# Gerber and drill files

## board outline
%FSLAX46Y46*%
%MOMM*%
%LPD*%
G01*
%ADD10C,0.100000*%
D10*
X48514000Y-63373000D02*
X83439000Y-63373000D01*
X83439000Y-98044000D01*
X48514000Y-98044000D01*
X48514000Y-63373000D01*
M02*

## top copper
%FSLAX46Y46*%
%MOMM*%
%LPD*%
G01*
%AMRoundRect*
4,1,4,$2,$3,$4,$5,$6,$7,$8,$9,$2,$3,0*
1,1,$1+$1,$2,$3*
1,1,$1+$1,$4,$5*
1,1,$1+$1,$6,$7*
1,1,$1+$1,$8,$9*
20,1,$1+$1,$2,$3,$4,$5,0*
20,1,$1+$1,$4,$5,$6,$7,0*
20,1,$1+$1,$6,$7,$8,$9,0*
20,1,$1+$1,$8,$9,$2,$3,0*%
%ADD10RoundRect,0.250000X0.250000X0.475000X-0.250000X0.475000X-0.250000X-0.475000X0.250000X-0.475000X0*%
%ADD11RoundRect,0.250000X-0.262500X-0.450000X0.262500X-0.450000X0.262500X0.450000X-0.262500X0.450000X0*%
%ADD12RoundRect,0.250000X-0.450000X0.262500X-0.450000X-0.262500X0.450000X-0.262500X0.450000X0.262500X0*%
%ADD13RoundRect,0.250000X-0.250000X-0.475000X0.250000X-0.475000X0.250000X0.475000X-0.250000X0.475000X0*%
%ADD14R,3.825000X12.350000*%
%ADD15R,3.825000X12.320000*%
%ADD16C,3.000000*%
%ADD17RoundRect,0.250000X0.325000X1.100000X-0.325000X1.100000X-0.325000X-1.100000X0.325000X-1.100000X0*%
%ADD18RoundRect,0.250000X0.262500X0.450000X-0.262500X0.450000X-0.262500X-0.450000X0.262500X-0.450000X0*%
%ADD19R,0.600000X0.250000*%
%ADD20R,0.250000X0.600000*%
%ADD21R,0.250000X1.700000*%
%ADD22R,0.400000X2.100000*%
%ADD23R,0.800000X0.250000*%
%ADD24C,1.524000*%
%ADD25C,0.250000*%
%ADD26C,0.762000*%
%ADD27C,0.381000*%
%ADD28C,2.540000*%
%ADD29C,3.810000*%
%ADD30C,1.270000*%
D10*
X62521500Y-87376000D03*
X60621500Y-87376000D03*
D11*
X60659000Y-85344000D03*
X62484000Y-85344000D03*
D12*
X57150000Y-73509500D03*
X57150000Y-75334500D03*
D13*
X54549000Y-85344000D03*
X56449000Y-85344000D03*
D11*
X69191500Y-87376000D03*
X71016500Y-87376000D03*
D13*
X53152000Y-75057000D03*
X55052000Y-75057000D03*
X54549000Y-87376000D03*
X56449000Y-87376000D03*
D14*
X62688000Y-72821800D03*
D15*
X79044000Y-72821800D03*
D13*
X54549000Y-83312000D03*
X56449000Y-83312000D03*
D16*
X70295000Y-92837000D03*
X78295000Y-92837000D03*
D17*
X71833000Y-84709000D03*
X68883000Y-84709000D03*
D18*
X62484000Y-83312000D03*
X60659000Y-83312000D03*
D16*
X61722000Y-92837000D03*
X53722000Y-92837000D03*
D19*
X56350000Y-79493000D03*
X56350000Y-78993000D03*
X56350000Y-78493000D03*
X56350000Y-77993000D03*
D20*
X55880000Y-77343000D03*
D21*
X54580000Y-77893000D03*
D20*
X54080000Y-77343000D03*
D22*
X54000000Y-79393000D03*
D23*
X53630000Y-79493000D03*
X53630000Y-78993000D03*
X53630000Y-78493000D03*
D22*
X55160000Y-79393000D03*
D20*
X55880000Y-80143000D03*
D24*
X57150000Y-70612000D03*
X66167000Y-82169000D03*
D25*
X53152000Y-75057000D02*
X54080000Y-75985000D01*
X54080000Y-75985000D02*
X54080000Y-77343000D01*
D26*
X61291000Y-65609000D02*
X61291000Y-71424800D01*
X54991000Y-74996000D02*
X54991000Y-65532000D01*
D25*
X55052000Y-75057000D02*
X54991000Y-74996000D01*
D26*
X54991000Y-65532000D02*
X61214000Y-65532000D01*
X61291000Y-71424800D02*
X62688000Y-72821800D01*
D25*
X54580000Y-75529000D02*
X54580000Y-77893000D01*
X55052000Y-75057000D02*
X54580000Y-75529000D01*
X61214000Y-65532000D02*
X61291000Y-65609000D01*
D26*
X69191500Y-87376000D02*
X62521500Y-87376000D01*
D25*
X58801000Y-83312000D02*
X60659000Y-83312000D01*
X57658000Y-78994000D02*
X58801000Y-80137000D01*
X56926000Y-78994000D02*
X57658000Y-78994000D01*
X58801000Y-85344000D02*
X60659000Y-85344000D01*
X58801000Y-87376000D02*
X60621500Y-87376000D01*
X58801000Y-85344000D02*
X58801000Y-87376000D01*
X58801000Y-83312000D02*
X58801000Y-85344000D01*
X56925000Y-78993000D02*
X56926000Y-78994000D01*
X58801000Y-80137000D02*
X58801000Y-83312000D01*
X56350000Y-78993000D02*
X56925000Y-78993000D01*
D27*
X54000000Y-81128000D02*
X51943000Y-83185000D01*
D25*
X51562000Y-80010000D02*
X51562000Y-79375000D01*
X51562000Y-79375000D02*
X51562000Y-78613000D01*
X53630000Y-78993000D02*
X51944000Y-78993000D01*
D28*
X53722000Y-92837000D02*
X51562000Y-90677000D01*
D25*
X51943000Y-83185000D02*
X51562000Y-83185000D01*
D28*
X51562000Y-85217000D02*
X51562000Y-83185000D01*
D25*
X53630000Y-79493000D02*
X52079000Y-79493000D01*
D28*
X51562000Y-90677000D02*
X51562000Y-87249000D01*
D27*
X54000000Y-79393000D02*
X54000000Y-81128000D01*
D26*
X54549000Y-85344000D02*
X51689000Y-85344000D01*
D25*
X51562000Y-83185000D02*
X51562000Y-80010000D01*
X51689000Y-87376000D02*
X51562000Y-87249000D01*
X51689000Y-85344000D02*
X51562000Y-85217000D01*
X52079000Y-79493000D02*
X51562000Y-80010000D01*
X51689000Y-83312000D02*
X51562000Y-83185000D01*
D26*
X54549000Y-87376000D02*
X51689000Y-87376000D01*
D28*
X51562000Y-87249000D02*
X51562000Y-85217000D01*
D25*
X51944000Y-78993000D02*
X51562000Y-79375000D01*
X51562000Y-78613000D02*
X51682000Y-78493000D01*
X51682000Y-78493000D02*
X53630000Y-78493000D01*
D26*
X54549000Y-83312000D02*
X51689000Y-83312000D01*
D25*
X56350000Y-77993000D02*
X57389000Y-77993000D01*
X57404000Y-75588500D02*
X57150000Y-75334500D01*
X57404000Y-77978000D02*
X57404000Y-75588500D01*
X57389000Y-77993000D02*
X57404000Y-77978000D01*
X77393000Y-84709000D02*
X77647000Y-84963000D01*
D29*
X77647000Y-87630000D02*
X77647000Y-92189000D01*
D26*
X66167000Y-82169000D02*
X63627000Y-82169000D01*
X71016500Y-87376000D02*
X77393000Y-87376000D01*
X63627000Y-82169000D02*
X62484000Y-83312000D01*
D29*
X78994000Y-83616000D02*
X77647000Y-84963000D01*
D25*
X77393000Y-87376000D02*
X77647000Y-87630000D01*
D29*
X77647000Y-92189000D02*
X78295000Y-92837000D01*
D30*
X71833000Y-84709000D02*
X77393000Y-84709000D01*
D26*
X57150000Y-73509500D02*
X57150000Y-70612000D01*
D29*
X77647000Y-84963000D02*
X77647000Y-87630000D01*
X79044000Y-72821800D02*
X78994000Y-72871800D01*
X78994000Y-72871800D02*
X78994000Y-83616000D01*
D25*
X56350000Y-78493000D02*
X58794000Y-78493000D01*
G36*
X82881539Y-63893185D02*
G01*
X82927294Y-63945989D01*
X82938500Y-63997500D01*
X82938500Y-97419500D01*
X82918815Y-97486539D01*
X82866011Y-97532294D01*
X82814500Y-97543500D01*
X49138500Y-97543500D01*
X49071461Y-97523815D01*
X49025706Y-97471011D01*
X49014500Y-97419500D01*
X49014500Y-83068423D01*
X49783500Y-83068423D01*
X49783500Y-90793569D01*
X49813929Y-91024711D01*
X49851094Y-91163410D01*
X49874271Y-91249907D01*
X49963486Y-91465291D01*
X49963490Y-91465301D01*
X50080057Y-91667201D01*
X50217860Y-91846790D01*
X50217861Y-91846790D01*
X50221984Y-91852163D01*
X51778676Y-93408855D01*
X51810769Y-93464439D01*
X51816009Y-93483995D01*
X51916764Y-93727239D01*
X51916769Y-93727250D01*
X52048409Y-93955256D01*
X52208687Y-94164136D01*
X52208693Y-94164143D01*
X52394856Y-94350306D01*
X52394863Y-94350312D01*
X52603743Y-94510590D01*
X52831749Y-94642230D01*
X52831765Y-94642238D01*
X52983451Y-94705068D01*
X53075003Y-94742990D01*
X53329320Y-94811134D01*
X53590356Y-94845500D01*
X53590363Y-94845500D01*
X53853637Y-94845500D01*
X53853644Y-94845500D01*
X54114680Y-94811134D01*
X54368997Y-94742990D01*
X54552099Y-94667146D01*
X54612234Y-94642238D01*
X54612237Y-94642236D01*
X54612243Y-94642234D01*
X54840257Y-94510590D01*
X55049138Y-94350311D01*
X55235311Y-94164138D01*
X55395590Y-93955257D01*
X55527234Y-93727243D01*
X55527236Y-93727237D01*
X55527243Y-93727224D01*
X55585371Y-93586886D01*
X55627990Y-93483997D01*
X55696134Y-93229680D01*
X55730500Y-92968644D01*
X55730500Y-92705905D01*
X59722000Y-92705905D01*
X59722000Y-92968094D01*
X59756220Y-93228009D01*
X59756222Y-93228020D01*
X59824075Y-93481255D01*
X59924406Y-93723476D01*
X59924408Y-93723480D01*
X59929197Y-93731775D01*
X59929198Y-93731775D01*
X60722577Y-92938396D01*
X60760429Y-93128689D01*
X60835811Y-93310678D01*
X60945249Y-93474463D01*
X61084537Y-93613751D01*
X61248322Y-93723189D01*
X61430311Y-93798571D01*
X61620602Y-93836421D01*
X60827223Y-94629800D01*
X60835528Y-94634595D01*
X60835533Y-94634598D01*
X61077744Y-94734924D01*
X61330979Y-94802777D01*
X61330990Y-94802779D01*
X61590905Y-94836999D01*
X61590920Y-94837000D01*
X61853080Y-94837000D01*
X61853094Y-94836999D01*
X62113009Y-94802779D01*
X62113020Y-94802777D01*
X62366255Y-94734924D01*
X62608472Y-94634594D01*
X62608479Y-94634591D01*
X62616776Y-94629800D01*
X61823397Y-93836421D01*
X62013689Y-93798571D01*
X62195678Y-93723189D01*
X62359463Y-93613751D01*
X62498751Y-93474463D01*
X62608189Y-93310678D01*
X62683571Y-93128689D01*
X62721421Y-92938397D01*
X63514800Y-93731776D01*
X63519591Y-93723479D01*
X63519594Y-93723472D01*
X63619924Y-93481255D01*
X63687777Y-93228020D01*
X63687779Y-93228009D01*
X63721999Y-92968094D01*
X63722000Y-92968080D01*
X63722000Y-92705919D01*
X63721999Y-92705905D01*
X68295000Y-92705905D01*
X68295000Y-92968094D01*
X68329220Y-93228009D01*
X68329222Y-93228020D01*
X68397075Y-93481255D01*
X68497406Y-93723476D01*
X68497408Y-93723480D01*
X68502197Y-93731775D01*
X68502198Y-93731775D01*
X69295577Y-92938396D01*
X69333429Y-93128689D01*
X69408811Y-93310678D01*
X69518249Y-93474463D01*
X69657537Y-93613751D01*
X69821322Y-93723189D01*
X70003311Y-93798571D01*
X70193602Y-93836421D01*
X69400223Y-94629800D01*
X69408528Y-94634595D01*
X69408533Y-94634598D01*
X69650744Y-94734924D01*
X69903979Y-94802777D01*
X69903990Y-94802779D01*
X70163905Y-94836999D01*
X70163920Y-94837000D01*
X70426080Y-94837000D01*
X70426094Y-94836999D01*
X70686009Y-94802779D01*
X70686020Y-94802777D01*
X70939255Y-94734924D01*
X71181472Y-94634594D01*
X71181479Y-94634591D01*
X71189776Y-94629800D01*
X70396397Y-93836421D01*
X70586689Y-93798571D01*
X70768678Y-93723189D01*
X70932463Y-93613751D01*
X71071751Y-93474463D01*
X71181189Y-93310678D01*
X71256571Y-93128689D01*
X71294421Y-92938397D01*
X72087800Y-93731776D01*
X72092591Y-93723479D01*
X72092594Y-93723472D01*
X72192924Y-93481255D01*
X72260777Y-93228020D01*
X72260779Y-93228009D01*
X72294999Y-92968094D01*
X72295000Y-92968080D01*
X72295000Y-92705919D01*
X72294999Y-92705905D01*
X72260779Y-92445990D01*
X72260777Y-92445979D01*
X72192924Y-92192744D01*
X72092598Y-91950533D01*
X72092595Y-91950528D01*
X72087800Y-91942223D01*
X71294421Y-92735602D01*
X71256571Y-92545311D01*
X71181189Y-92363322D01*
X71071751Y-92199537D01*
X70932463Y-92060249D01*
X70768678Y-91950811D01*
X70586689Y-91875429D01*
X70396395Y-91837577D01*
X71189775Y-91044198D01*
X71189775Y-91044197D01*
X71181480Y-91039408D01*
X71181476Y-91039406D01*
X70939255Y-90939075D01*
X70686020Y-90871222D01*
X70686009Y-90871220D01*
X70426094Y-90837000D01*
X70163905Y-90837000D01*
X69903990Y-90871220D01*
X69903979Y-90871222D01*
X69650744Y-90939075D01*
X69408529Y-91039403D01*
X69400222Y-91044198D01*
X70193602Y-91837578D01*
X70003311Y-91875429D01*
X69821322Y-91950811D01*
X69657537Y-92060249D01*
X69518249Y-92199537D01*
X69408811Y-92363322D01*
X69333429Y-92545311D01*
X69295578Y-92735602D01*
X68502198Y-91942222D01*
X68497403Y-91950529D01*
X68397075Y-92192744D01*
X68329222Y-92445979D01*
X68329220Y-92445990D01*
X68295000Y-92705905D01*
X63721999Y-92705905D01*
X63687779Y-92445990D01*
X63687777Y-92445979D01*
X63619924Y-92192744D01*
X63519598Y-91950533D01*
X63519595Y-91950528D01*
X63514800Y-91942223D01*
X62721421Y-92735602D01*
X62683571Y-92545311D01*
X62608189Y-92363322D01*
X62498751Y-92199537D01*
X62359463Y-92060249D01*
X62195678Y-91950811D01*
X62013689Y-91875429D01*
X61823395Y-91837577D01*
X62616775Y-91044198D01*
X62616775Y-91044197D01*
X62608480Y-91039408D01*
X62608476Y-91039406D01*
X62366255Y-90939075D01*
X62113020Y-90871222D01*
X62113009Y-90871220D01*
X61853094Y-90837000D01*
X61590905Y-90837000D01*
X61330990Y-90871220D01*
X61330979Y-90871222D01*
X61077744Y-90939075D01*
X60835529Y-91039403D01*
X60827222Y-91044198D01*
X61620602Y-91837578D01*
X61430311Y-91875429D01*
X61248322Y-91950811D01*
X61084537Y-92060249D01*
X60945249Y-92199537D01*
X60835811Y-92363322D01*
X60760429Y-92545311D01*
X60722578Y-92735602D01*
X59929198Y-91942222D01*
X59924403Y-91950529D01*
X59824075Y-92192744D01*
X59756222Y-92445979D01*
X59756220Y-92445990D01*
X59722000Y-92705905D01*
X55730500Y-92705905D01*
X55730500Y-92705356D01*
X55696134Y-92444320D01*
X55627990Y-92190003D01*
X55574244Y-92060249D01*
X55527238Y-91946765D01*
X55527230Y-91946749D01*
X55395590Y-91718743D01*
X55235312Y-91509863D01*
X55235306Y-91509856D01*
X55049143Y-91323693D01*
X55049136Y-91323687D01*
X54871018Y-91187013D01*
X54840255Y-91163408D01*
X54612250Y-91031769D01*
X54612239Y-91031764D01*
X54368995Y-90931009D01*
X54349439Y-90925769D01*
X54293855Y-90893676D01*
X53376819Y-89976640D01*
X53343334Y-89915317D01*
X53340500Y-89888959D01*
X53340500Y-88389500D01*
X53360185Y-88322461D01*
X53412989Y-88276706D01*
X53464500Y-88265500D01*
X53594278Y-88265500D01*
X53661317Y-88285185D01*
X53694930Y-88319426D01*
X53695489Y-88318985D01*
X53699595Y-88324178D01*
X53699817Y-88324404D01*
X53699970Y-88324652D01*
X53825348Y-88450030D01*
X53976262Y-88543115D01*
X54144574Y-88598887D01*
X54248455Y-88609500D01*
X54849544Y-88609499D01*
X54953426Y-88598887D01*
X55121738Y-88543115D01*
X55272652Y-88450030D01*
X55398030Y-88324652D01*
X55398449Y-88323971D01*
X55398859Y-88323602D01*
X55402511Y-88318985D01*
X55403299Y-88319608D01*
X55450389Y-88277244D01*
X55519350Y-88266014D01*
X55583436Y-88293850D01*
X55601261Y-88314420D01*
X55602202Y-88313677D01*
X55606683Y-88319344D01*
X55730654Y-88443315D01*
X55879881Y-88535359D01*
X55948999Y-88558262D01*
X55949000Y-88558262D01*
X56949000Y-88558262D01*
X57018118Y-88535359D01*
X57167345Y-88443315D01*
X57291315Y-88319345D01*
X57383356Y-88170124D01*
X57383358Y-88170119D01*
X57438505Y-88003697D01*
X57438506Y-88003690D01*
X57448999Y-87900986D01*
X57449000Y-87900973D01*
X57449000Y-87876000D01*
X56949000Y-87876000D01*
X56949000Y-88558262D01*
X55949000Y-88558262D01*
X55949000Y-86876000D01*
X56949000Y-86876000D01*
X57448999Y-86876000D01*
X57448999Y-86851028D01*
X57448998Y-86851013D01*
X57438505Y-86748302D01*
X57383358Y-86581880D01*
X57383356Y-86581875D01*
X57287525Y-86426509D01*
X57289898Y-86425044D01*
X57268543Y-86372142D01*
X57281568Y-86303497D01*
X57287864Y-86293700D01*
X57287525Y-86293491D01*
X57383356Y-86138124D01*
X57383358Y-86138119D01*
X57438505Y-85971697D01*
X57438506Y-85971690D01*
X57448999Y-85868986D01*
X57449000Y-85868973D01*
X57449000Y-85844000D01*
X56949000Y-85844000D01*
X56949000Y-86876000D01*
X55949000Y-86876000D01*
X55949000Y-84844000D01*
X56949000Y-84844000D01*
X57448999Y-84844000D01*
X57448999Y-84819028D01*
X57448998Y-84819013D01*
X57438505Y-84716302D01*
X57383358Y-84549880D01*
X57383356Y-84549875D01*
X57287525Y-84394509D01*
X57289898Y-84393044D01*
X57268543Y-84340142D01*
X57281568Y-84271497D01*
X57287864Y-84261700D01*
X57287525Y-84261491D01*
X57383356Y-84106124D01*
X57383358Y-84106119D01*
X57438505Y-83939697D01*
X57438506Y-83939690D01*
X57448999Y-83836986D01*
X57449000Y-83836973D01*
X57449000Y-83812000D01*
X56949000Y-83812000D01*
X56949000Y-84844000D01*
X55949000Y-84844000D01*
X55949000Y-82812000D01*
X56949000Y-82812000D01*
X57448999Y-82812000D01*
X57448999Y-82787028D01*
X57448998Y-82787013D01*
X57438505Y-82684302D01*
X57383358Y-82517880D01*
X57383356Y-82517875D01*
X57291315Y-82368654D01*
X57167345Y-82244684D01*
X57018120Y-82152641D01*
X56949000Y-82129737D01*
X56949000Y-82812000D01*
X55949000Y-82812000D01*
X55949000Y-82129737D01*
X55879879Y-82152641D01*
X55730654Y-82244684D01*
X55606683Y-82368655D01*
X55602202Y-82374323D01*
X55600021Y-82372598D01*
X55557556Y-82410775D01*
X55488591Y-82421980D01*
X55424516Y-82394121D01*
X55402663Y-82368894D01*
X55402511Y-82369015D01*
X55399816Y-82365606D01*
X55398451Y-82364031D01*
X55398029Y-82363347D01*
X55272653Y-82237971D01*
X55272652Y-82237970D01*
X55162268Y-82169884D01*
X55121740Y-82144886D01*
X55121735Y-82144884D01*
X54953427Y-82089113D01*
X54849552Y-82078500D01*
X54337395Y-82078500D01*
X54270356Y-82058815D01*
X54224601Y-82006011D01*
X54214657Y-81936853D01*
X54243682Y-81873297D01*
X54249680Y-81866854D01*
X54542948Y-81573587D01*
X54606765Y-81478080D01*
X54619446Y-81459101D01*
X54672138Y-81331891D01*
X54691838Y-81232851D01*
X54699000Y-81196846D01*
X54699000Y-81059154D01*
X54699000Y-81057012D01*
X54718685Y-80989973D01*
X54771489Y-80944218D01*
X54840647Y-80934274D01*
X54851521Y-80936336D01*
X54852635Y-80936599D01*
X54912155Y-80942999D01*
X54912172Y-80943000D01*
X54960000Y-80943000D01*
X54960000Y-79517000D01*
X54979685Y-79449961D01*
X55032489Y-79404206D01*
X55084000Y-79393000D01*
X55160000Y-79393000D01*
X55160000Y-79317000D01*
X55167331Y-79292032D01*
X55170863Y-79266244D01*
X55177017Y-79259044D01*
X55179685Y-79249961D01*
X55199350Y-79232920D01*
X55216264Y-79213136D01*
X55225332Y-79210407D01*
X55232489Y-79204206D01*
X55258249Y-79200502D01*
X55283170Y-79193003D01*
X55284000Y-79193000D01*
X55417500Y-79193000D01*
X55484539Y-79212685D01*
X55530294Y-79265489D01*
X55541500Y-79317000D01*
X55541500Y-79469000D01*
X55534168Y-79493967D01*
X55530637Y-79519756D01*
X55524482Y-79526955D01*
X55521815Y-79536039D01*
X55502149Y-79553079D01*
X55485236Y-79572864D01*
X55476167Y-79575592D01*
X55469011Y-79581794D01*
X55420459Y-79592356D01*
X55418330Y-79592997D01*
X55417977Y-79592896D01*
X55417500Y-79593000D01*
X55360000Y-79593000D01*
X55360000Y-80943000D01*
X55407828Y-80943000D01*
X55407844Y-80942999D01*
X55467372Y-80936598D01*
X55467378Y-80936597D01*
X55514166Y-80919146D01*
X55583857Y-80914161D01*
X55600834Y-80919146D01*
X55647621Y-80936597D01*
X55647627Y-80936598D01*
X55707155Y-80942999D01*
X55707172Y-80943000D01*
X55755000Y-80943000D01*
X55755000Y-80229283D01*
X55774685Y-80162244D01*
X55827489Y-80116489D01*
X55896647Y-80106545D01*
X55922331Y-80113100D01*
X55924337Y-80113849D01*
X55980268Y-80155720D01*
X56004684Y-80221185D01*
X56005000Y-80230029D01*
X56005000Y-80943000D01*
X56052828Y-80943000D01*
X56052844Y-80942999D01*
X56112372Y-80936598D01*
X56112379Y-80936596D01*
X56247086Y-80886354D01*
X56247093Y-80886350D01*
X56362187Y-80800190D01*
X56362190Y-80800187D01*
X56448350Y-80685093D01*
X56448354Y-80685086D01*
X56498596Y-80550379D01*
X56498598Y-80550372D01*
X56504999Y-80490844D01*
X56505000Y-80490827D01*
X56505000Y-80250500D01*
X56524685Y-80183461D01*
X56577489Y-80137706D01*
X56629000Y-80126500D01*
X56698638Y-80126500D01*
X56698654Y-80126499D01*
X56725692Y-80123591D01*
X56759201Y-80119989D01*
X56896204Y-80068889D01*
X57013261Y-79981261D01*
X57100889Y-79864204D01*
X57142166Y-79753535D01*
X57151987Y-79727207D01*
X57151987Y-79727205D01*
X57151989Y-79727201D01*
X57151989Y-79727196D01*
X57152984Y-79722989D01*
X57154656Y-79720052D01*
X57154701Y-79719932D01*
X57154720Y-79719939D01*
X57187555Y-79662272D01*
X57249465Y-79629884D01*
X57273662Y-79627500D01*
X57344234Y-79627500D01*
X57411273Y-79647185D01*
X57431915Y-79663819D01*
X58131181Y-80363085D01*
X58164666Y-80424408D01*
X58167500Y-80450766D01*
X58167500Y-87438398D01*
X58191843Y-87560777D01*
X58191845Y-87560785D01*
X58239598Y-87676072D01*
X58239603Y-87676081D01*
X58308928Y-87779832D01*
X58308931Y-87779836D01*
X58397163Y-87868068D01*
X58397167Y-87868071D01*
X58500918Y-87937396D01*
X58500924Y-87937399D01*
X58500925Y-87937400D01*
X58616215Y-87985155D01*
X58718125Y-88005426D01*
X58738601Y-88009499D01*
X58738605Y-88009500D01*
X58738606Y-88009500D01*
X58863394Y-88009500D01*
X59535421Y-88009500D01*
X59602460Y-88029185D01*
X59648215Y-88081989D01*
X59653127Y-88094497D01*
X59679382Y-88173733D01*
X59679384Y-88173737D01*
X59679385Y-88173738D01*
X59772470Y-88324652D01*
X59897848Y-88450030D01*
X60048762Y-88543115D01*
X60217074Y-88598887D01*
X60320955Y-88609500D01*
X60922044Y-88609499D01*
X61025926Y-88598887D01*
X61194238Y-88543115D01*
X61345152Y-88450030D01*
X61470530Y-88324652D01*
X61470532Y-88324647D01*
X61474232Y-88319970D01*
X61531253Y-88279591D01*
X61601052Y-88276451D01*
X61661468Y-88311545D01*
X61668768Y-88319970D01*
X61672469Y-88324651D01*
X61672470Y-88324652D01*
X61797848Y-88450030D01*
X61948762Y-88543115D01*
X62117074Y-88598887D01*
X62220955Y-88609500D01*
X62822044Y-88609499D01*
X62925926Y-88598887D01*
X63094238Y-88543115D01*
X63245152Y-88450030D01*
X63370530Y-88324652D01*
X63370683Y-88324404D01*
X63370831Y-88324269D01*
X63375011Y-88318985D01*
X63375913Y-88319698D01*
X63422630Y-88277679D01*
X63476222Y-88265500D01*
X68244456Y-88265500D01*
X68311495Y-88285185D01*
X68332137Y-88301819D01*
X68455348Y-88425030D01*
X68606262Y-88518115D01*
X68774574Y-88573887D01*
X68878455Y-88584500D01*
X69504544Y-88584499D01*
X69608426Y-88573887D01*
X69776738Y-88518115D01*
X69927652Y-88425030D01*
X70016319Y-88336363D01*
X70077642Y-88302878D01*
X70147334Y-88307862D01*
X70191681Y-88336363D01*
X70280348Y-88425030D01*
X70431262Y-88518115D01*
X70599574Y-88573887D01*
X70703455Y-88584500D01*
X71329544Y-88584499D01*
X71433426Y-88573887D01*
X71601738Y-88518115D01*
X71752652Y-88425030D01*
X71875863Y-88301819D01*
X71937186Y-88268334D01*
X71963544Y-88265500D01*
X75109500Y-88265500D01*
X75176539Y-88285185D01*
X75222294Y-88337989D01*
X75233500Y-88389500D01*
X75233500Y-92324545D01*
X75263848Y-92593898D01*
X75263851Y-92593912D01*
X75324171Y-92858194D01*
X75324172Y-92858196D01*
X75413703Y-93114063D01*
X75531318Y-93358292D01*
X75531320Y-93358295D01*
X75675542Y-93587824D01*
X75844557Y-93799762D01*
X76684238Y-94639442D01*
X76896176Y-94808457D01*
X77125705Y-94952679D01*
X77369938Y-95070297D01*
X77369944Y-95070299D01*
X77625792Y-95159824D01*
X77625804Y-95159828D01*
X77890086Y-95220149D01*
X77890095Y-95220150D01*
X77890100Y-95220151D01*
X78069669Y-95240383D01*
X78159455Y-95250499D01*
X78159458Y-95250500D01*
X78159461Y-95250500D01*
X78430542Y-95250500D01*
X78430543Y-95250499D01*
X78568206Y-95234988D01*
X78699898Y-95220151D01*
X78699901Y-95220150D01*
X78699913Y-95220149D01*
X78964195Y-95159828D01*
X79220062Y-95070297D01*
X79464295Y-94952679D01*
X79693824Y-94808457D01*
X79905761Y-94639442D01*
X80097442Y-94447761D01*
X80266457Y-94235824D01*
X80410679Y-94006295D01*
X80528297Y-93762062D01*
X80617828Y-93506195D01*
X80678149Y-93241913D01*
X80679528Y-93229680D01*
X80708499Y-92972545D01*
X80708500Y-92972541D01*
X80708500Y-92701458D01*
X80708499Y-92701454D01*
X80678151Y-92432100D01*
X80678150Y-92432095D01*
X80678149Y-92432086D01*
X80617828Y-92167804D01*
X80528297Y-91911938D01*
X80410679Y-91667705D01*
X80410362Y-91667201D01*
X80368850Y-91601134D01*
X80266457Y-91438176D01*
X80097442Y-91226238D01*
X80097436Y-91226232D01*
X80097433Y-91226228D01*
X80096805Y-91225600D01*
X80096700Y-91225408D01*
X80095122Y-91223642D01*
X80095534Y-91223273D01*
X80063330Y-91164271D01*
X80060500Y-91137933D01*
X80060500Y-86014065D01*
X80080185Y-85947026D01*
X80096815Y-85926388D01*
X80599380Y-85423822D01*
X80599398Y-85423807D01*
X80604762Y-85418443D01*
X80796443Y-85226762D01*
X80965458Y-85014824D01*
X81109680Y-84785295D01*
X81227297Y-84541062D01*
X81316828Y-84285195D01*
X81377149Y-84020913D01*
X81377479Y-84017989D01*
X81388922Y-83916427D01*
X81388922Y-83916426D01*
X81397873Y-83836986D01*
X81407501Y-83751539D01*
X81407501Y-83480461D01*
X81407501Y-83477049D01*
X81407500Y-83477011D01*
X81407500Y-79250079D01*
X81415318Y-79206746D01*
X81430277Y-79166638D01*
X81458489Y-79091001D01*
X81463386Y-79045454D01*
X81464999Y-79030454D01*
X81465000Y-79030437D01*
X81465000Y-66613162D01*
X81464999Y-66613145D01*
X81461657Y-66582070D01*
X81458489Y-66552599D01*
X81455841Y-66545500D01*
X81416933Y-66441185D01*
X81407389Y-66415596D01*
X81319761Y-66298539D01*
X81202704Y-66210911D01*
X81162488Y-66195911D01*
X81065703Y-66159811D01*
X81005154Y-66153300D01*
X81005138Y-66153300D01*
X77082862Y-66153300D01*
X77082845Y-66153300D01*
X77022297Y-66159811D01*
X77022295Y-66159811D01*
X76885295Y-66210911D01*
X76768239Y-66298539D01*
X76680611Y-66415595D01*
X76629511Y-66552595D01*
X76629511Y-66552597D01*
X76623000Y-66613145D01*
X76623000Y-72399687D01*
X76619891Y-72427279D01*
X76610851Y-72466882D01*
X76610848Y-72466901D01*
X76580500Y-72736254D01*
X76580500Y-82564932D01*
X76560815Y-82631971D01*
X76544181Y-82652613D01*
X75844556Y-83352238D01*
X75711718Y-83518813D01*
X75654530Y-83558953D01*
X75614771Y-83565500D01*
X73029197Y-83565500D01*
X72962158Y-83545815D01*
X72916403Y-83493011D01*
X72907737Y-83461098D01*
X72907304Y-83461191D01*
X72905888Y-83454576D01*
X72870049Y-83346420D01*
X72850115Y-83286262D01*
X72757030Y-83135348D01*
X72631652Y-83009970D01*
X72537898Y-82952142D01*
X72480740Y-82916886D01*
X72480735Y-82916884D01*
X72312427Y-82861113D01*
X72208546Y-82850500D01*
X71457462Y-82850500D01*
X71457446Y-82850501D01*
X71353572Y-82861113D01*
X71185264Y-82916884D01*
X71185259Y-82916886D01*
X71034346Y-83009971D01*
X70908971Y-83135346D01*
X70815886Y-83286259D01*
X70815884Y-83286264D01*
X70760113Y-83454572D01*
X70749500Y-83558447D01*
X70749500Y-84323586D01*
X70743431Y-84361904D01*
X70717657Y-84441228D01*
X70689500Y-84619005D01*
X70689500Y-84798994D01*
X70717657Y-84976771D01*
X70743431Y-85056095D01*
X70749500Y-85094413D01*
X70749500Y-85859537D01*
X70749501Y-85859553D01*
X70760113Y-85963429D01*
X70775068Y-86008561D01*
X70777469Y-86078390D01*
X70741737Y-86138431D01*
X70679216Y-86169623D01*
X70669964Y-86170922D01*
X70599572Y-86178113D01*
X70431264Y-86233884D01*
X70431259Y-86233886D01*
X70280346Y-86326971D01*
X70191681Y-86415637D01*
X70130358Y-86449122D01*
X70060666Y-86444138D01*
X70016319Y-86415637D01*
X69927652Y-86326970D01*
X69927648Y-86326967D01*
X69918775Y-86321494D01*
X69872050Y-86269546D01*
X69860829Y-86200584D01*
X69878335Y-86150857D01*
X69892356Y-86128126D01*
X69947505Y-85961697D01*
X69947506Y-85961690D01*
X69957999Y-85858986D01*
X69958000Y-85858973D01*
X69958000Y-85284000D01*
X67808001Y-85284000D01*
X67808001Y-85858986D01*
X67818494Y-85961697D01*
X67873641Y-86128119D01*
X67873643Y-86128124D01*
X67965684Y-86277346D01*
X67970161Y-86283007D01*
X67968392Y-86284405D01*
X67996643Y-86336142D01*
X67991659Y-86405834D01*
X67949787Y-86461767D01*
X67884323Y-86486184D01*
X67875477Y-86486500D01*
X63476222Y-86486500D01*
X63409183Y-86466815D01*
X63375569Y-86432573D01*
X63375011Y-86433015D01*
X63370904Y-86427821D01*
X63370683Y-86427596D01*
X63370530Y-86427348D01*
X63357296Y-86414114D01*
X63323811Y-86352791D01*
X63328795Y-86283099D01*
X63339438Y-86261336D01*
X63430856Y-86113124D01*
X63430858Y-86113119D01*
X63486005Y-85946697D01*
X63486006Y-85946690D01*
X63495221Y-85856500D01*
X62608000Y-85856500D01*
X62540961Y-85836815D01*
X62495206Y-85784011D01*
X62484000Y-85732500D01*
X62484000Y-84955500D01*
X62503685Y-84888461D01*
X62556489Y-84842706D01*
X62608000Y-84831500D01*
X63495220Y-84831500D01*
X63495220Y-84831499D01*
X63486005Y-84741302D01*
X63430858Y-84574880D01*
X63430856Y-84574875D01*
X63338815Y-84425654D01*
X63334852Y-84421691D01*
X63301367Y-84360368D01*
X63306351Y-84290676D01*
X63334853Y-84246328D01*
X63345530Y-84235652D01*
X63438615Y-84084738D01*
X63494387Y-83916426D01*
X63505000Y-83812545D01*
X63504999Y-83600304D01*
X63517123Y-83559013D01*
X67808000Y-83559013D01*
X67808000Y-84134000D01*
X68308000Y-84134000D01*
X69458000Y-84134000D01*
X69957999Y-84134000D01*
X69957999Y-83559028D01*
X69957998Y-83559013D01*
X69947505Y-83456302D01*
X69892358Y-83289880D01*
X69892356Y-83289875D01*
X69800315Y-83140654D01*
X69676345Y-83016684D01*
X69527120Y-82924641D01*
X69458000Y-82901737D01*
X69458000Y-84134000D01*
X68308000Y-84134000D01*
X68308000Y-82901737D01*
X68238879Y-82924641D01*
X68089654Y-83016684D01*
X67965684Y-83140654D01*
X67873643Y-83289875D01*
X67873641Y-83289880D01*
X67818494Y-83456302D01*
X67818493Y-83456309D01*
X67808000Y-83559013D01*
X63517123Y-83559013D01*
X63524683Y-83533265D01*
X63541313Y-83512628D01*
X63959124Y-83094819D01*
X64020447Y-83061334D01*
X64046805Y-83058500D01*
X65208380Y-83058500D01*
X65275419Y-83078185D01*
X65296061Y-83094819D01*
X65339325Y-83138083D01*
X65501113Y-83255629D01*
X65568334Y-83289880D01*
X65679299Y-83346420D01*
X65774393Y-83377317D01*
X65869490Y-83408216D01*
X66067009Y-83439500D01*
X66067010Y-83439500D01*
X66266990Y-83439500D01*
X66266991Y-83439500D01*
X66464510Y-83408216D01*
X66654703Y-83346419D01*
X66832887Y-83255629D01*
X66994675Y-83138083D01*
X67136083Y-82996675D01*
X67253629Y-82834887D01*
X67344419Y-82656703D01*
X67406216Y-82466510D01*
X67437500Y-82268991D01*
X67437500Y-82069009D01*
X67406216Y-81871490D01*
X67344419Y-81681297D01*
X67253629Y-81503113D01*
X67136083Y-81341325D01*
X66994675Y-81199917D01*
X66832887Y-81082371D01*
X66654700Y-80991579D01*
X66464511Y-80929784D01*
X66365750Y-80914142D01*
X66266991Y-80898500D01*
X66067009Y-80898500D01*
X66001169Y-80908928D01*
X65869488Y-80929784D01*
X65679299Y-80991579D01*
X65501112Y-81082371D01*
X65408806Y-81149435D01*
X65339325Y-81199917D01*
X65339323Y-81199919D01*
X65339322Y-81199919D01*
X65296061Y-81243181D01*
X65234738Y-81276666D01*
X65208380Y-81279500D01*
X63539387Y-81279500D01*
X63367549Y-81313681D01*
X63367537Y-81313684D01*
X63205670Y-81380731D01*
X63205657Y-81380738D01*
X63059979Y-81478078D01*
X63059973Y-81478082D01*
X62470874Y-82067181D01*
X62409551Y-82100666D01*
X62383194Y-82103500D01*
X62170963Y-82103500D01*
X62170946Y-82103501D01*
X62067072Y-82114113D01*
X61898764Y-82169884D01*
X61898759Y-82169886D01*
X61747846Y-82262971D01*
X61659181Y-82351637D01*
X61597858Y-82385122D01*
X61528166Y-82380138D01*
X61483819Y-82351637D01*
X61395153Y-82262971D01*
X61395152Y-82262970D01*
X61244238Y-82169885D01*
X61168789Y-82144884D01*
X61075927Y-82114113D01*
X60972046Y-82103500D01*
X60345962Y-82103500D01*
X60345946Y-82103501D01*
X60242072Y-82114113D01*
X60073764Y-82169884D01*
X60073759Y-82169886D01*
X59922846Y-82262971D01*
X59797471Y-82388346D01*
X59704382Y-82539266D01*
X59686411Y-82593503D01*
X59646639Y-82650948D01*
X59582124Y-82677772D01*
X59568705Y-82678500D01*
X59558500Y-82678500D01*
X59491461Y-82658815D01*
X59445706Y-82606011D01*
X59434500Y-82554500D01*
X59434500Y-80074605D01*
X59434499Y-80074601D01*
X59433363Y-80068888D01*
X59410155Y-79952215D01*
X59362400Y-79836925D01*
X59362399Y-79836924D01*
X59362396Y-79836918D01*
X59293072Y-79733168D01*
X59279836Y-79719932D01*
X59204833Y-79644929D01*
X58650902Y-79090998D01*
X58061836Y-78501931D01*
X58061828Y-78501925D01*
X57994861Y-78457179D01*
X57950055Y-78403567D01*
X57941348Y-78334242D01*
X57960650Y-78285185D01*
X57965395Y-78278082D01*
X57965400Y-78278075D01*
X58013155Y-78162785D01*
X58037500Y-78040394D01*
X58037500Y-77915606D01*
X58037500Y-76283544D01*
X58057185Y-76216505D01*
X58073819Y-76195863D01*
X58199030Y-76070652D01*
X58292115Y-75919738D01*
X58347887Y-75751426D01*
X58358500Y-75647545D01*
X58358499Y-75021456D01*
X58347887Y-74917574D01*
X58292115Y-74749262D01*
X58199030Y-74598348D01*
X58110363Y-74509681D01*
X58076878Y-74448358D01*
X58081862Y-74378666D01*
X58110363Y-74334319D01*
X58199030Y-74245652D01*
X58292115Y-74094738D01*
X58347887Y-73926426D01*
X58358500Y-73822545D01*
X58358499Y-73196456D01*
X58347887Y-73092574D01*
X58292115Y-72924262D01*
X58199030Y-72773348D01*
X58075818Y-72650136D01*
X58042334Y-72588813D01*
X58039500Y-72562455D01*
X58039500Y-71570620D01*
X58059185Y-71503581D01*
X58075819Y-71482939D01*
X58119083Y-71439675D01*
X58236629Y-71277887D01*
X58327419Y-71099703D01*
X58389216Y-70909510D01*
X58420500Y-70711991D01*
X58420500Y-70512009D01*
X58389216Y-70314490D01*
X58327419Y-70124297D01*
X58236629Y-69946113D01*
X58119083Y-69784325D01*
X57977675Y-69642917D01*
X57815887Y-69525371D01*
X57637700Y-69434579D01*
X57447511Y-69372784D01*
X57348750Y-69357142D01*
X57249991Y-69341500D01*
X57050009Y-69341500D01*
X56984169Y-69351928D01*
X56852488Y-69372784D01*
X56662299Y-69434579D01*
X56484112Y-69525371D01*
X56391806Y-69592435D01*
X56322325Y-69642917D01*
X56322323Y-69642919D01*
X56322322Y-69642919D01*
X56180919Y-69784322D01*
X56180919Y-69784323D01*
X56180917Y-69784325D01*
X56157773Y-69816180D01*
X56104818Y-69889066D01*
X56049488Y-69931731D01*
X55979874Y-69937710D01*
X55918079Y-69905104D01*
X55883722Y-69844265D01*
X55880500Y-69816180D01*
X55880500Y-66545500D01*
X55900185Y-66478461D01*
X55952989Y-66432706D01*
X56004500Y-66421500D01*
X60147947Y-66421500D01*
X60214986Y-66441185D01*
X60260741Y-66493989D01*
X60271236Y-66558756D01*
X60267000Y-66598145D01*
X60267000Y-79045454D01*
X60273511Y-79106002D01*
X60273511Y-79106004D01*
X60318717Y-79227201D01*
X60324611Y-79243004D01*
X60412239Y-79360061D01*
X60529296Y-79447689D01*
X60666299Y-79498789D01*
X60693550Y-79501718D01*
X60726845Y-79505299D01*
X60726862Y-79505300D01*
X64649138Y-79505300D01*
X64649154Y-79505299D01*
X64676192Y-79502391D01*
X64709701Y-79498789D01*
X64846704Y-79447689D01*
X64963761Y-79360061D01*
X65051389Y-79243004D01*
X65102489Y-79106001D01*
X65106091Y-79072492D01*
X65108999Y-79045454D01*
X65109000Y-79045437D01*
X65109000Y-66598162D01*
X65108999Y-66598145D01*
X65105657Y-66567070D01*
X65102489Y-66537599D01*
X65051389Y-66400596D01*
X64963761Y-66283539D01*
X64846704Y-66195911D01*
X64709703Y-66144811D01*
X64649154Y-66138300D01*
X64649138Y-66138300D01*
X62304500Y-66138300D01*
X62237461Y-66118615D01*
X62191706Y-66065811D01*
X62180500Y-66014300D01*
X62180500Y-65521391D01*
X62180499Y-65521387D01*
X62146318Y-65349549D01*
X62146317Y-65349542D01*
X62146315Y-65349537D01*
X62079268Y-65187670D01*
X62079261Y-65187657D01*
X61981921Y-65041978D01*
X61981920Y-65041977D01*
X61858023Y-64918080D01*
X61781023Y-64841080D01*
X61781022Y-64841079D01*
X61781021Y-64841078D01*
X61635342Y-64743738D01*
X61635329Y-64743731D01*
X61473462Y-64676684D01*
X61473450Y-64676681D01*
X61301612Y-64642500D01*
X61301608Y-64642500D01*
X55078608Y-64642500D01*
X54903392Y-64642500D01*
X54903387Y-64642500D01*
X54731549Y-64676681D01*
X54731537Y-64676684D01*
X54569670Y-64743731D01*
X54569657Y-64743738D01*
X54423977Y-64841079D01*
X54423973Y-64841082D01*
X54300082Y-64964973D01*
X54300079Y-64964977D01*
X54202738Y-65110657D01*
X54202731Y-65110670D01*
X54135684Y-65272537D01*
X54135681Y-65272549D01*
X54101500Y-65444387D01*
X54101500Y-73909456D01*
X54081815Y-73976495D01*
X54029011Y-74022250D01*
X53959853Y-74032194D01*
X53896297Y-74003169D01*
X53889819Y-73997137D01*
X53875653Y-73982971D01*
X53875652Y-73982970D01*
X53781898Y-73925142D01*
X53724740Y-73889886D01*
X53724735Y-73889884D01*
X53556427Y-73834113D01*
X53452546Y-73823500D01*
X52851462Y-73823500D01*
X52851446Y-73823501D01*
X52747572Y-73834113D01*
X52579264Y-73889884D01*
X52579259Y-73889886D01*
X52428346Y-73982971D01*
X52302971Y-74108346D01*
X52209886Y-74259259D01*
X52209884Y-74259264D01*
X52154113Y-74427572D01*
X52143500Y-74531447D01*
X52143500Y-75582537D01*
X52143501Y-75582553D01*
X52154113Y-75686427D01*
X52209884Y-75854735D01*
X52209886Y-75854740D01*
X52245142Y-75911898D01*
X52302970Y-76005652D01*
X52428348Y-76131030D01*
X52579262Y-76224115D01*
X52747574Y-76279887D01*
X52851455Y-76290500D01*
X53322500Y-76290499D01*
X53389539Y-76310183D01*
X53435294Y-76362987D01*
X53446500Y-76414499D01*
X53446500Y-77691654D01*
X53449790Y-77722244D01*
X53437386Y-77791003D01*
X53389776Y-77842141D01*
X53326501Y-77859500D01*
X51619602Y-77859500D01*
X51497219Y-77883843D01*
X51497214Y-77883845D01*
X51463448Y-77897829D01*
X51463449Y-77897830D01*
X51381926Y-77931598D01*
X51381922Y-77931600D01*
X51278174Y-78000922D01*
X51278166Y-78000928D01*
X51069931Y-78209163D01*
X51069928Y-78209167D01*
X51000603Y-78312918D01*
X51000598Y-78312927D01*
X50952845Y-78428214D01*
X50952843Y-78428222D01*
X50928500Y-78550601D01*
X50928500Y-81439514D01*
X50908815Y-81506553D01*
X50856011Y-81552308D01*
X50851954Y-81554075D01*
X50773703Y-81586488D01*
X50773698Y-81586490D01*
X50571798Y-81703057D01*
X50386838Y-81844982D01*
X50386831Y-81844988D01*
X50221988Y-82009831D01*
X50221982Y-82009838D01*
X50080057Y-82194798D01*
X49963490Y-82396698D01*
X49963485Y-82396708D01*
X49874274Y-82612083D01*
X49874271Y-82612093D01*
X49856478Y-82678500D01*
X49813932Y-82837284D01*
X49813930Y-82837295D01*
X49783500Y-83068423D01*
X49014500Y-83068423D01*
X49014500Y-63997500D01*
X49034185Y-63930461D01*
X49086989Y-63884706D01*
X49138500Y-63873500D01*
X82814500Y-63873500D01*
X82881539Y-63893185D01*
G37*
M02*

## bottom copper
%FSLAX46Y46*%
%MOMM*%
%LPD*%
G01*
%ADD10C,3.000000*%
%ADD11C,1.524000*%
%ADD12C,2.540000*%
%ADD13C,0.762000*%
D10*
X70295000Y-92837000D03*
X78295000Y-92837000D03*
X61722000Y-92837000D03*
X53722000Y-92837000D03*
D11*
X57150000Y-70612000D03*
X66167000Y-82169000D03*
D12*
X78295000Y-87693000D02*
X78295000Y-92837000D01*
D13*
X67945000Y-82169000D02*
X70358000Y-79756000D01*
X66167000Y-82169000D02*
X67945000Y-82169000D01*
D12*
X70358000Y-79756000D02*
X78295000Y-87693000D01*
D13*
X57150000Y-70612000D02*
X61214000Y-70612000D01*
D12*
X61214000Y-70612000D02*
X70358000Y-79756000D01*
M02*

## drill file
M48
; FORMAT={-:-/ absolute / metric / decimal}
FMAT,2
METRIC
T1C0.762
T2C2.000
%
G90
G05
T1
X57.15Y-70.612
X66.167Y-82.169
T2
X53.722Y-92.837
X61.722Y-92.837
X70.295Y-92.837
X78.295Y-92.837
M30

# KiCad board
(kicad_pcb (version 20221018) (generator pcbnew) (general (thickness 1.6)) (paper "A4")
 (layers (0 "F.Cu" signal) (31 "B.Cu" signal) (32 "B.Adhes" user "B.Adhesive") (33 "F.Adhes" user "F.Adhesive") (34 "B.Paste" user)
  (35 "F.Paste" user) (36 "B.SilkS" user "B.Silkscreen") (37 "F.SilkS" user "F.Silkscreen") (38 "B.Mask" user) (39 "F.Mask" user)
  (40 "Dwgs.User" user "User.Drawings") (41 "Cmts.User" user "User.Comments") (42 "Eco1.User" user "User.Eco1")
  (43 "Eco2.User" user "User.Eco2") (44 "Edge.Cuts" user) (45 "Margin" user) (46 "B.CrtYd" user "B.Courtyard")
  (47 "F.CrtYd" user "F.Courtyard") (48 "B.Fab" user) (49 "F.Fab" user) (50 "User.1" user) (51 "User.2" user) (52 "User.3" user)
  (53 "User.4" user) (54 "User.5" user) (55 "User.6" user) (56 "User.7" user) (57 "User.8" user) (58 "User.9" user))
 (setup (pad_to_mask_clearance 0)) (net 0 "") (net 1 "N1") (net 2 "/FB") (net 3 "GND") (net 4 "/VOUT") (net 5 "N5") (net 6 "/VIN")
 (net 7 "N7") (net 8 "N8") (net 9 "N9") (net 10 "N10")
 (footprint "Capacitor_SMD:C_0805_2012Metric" (layer "F.Cu") (at 61.5715 87.376 180)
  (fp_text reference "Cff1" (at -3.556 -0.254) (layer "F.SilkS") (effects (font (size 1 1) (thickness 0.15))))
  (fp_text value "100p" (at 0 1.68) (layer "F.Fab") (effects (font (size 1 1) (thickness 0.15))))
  (pad "1" smd roundrect (at -0.95 0 180) (size 1 1.45) (layers "F.Cu" "F.Paste" "F.Mask") (roundrect_rratio 0.25) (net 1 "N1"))
  (pad "2" smd roundrect (at 0.95 0 180) (size 1 1.45) (layers "F.Cu" "F.Paste" "F.Mask") (roundrect_rratio 0.25) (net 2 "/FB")))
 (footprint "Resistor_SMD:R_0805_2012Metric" (layer "F.Cu") (at 61.5715 85.344)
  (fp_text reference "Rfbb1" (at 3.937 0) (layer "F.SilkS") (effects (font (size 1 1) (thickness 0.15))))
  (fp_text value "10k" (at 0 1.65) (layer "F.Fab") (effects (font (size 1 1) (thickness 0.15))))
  (pad "1" smd roundrect (at -0.9125 0) (size 1.025 1.4) (layers "F.Cu" "F.Paste" "F.Mask") (roundrect_rratio 0.243902) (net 2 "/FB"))
  (pad "2" smd roundrect (at 0.9125 0) (size 1.025 1.4) (layers "F.Cu" "F.Paste" "F.Mask") (roundrect_rratio 0.243902) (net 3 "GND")))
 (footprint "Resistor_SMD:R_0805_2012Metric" (layer "F.Cu") (at 57.15 74.422 -90)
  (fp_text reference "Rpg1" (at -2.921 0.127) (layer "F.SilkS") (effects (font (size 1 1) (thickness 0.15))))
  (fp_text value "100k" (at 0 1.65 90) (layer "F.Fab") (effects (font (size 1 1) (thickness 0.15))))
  (pad "1" smd roundrect (at -0.9125 0 270) (size 1.025 1.4) (layers "F.Cu" "F.Paste" "F.Mask") (roundrect_rratio 0.243902) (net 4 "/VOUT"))
  (pad "2" smd roundrect (at 0.9125 0 270) (size 1.025 1.4) (layers "F.Cu" "F.Paste" "F.Mask") (roundrect_rratio 0.243902) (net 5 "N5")))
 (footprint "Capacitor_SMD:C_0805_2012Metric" (layer "F.Cu") (at 55.499 85.344)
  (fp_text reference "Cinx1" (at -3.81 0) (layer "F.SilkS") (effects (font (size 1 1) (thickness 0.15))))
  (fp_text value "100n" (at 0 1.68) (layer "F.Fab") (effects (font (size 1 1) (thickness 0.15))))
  (pad "1" smd roundrect (at -0.95 0) (size 1 1.45) (layers "F.Cu" "F.Paste" "F.Mask") (roundrect_rratio 0.25) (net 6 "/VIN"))
  (pad "2" smd roundrect (at 0.95 0) (size 1 1.45) (layers "F.Cu" "F.Paste" "F.Mask") (roundrect_rratio 0.25) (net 3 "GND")))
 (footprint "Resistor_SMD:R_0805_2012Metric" (layer "F.Cu") (at 70.104 87.376)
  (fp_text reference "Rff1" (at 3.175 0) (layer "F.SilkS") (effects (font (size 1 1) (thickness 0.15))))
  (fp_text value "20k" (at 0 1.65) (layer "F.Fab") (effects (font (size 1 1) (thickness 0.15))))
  (pad "1" smd roundrect (at -0.9125 0) (size 1.025 1.4) (layers "F.Cu" "F.Paste" "F.Mask") (roundrect_rratio 0.243902) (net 1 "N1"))
  (pad "2" smd roundrect (at 0.9125 0) (size 1.025 1.4) (layers "F.Cu" "F.Paste" "F.Mask") (roundrect_rratio 0.243902) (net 4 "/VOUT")))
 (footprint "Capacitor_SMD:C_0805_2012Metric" (layer "F.Cu") (at 54.102 75.057)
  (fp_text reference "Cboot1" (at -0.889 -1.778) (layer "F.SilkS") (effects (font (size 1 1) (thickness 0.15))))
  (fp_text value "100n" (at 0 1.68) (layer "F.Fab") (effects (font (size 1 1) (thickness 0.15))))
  (pad "1" smd roundrect (at -0.95 0) (size 1 1.45) (layers "F.Cu" "F.Paste" "F.Mask") (roundrect_rratio 0.25) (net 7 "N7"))
  (pad "2" smd roundrect (at 0.95 0) (size 1 1.45) (layers "F.Cu" "F.Paste" "F.Mask") (roundrect_rratio 0.25) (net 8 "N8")))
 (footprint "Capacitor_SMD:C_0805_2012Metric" (layer "F.Cu") (at 55.499 87.376)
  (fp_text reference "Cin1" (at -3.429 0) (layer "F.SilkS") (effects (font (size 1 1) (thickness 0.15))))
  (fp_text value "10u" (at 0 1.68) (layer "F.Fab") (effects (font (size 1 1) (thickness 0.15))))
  (pad "1" smd roundrect (at -0.95 0) (size 1 1.45) (layers "F.Cu" "F.Paste" "F.Mask") (roundrect_rratio 0.25) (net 6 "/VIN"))
  (pad "2" smd roundrect (at 0.95 0) (size 1 1.45) (layers "F.Cu" "F.Paste" "F.Mask") (roundrect_rratio 0.25) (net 3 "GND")))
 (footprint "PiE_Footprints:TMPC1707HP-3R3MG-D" (layer "F.Cu") (at 70.866 65.786)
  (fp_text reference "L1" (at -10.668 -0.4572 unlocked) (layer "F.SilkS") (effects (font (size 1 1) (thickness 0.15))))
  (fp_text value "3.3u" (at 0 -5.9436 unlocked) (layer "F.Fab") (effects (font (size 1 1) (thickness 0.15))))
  (pad "1" smd rect (at -8.178 7.0358) (size 3.825 12.35) (layers "F.Cu" "F.Paste" "F.Mask") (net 8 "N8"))
  (pad "2" smd rect (at 8.178 7.0358) (size 3.825 12.32) (layers "F.Cu" "F.Paste" "F.Mask") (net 4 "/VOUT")))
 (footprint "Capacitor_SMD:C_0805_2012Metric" (layer "F.Cu") (at 55.499 83.312)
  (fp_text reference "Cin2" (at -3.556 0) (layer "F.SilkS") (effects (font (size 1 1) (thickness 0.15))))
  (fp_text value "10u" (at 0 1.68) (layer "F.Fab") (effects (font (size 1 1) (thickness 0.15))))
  (pad "1" smd roundrect (at -0.95 0) (size 1 1.45) (layers "F.Cu" "F.Paste" "F.Mask") (roundrect_rratio 0.25) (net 6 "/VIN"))
  (pad "2" smd roundrect (at 0.95 0) (size 1 1.45) (layers "F.Cu" "F.Paste" "F.Mask") (roundrect_rratio 0.25) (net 3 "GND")))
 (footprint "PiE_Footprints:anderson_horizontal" (layer "F.Cu") (at 74.295 96.837 180)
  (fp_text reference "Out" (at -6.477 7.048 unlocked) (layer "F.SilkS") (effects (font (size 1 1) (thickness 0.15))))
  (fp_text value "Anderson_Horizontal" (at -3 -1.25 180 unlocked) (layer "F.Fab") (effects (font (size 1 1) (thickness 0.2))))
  (pad "1" thru_hole circle (at 4 4 180) (size 3 3) (drill 2) (layers "*.Cu" "*.Mask") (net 3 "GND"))
  (pad "2" thru_hole circle (at -4 4 180) (size 3 3) (drill 2) (layers "*.Cu" "*.Mask") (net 4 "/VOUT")))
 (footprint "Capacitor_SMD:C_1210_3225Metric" (layer "F.Cu") (at 70.358 84.709 180)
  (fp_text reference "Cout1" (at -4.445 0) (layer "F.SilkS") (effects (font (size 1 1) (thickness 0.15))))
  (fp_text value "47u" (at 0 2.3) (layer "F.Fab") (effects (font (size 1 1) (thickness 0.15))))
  (pad "1" smd roundrect (at -1.475 0 180) (size 1.15 2.7) (layers "F.Cu" "F.Paste" "F.Mask") (roundrect_rratio 0.217391) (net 4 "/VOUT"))
  (pad "2" smd roundrect (at 1.475 0 180) (size 1.15 2.7) (layers "F.Cu" "F.Paste" "F.Mask") (roundrect_rratio 0.217391) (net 3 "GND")))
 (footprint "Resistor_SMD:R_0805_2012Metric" (layer "F.Cu") (at 61.5715 83.312 180)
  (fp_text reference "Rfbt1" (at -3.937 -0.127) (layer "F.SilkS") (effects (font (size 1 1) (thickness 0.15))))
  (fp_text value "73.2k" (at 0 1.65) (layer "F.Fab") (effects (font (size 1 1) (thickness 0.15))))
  (pad "1" smd roundrect (at -0.9125 0 180) (size 1.025 1.4) (layers "F.Cu" "F.Paste" "F.Mask") (roundrect_rratio 0.243902) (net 4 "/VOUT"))
  (pad "2" smd roundrect (at 0.9125 0 180) (size 1.025 1.4) (layers "F.Cu" "F.Paste" "F.Mask") (roundrect_rratio 0.243902) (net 2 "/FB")))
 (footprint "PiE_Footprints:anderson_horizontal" (layer "F.Cu") (at 57.722 88.837)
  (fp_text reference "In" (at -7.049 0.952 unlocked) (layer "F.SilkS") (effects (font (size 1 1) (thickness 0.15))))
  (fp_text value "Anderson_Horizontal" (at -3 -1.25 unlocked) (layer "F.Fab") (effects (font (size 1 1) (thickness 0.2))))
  (pad "1" thru_hole circle (at 4 4) (size 3 3) (drill 2) (layers "*.Cu" "*.Mask") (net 3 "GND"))
  (pad "2" thru_hole circle (at -4 4) (size 3 3) (drill 2) (layers "*.Cu" "*.Mask") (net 6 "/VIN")))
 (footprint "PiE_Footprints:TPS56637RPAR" (layer "F.Cu") (at 54.99 85.0422 180)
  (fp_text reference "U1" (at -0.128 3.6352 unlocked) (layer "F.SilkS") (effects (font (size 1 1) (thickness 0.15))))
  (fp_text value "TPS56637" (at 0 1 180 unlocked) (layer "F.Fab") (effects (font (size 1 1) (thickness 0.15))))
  (pad "1" smd rect (at -1.36 5.5492 180) (size 0.6 0.25) (layers "F.Cu" "F.Paste" "F.Mask") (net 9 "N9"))
  (pad "2" smd rect (at -1.36 6.0492 180) (size 0.6 0.25) (layers "F.Cu" "F.Paste" "F.Mask") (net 2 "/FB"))
  (pad "3" smd rect (at -1.36 6.5492 180) (size 0.6 0.25) (layers "F.Cu" "F.Paste" "F.Mask") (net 3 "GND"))
  (pad "4" smd rect (at -1.36 7.0492 180) (size 0.6 0.25) (layers "F.Cu" "F.Paste" "F.Mask") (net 5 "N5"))
  (pad "5" smd rect (at -0.89 7.6992 90) (size 0.6 0.25) (layers "F.Cu" "F.Paste" "F.Mask") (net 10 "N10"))
  (pad "6" smd rect (at 0.41 7.1492 180) (size 0.25 1.7) (layers "F.Cu" "F.Paste" "F.Mask") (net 8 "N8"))
  (pad "7" smd rect (at 0.91 7.6992 90) (size 0.6 0.25) (layers "F.Cu" "F.Paste" "F.Mask") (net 7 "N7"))
  (pad "8" smd rect (at 0.99 5.6492 180) (size 0.4 2.1) (layers "F.Cu" "F.Paste" "F.Mask") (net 6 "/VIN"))
  (pad "8" smd rect (at 1.36 5.5492 180) (size 0.8 0.25) (layers "F.Cu" "F.Paste" "F.Mask") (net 6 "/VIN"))
  (pad "8" smd rect (at 1.36 6.0492 180) (size 0.8 0.25) (layers "F.Cu" "F.Paste" "F.Mask") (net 6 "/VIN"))
  (pad "8" smd rect (at 1.36 6.5492 180) (size 0.8 0.25) (layers "F.Cu" "F.Paste" "F.Mask") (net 6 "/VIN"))
  (pad "9" smd rect (at -0.17 5.6492 180) (size 0.4 2.1) (layers "F.Cu" "F.Paste" "F.Mask") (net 3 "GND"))
  (pad "10" smd rect (at -0.89 4.8992 90) (size 0.6 0.25) (layers "F.Cu" "F.Paste" "F.Mask") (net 3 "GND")))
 (gr_rect (start 48.514 63.373) (end 83.439 98.044) (stroke (width 0.1) (type default)) (fill none) (layer "Edge.Cuts"))
 (segment (start 53.152 75.057) (end 54.08 75.985) (width 0.25) (layer "F.Cu") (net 7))
 (segment (start 54.08 75.985) (end 54.08 77.343) (width 0.25) (layer "F.Cu") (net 7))
 (segment (start 61.291 65.609) (end 61.291 71.4248) (width 0.762) (layer "F.Cu") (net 8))
 (segment (start 54.991 74.996) (end 54.991 65.532) (width 0.762) (layer "F.Cu") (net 8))
 (segment (start 55.052 75.057) (end 54.991 74.996) (width 0.25) (layer "F.Cu") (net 8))
 (segment (start 54.991 65.532) (end 61.214 65.532) (width 0.762) (layer "F.Cu") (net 8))
 (segment (start 61.291 71.4248) (end 62.688 72.8218) (width 0.762) (layer "F.Cu") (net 8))
 (segment (start 54.58 75.529) (end 54.58 77.893) (width 0.25) (layer "F.Cu") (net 8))
 (segment (start 55.052 75.057) (end 54.58 75.529) (width 0.25) (layer "F.Cu") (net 8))
 (segment (start 61.214 65.532) (end 61.291 65.609) (width 0.25) (layer "F.Cu") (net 8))
 (segment (start 69.1915 87.376) (end 62.5215 87.376) (width 0.762) (layer "F.Cu") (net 1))
 (segment (start 58.801 83.312) (end 60.659 83.312) (width 0.25) (layer "F.Cu") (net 2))
 (segment (start 57.658 78.994) (end 58.801 80.137) (width 0.25) (layer "F.Cu") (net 2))
 (segment (start 56.926 78.994) (end 57.658 78.994) (width 0.25) (layer "F.Cu") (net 2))
 (segment (start 58.801 85.344) (end 60.659 85.344) (width 0.25) (layer "F.Cu") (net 2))
 (segment (start 58.801 87.376) (end 60.6215 87.376) (width 0.25) (layer "F.Cu") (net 2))
 (segment (start 58.801 85.344) (end 58.801 87.376) (width 0.25) (layer "F.Cu") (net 2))
 (segment (start 58.801 83.312) (end 58.801 85.344) (width 0.25) (layer "F.Cu") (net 2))
 (segment (start 56.925 78.993) (end 56.926 78.994) (width 0.25) (layer "F.Cu") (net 2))
 (segment (start 58.801 80.137) (end 58.801 83.312) (width 0.25) (layer "F.Cu") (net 2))
 (segment (start 56.35 78.993) (end 56.925 78.993) (width 0.25) (layer "F.Cu") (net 2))
 (segment (start 54 81.128) (end 51.943 83.185) (width 0.381) (layer "F.Cu") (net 6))
 (segment (start 51.562 80.01) (end 51.562 79.375) (width 0.25) (layer "F.Cu") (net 6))
 (segment (start 51.562 79.375) (end 51.562 78.613) (width 0.25) (layer "F.Cu") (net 6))
 (segment (start 53.63 78.993) (end 51.944 78.993) (width 0.25) (layer "F.Cu") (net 6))
 (segment (start 53.722 92.837) (end 51.562 90.677) (width 2.54) (layer "F.Cu") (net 6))
 (segment (start 51.943 83.185) (end 51.562 83.185) (width 0.25) (layer "F.Cu") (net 6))
 (segment (start 51.562 85.217) (end 51.562 83.185) (width 2.54) (layer "F.Cu") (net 6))
 (segment (start 53.63 79.493) (end 52.079 79.493) (width 0.25) (layer "F.Cu") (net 6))
 (segment (start 51.562 90.677) (end 51.562 87.249) (width 2.54) (layer "F.Cu") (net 6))
 (segment (start 54 79.393) (end 54 81.128) (width 0.381) (layer "F.Cu") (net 6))
 (segment (start 54.549 85.344) (end 51.689 85.344) (width 0.762) (layer "F.Cu") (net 6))
 (segment (start 51.562 83.185) (end 51.562 80.01) (width 0.25) (layer "F.Cu") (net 6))
 (segment (start 51.689 87.376) (end 51.562 87.249) (width 0.25) (layer "F.Cu") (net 6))
 (segment (start 51.689 85.344) (end 51.562 85.217) (width 0.25) (layer "F.Cu") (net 6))
 (segment (start 52.079 79.493) (end 51.562 80.01) (width 0.25) (layer "F.Cu") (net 6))
 (segment (start 51.689 83.312) (end 51.562 83.185) (width 0.25) (layer "F.Cu") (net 6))
 (segment (start 54.549 87.376) (end 51.689 87.376) (width 0.762) (layer "F.Cu") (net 6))
 (segment (start 51.562 87.249) (end 51.562 85.217) (width 2.54) (layer "F.Cu") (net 6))
 (segment (start 51.944 78.993) (end 51.562 79.375) (width 0.25) (layer "F.Cu") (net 6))
 (segment (start 51.562 78.613) (end 51.682 78.493) (width 0.25) (layer "F.Cu") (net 6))
 (segment (start 51.682 78.493) (end 53.63 78.493) (width 0.25) (layer "F.Cu") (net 6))
 (segment (start 54.549 83.312) (end 51.689 83.312) (width 0.762) (layer "F.Cu") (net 6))
 (segment (start 56.35 77.993) (end 57.389 77.993) (width 0.25) (layer "F.Cu") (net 5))
 (segment (start 57.404 75.5885) (end 57.15 75.3345) (width 0.25) (layer "F.Cu") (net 5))
 (segment (start 57.404 77.978) (end 57.404 75.5885) (width 0.25) (layer "F.Cu") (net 5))
 (segment (start 57.389 77.993) (end 57.404 77.978) (width 0.25) (layer "F.Cu") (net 5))
 (segment (start 77.393 84.709) (end 77.647 84.963) (width 0.25) (layer "F.Cu") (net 4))
 (segment (start 77.647 87.63) (end 77.647 92.189) (width 3.81) (layer "F.Cu") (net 4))
 (segment (start 66.167 82.169) (end 63.627 82.169) (width 0.762) (layer "F.Cu") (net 4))
 (segment (start 71.0165 87.376) (end 77.393 87.376) (width 0.762) (layer "F.Cu") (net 4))
 (segment (start 63.627 82.169) (end 62.484 83.312) (width 0.762) (layer "F.Cu") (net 4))
 (segment (start 78.994 83.616) (end 77.647 84.963) (width 3.81) (layer "F.Cu") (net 4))
 (segment (start 77.393 87.376) (end 77.647 87.63) (width 0.25) (layer "F.Cu") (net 4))
 (segment (start 77.647 92.189) (end 78.295 92.837) (width 3.81) (layer "F.Cu") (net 4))
 (segment (start 71.833 84.709) (end 77.393 84.709) (width 1.27) (layer "F.Cu") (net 4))
 (segment (start 57.15 73.5095) (end 57.15 70.612) (width 0.762) (layer "F.Cu") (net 4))
 (segment (start 77.647 84.963) (end 77.647 87.63) (width 3.81) (layer "F.Cu") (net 4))
 (segment (start 79.044 72.8218) (end 78.994 72.8718) (width 3.81) (layer "F.Cu") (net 4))
 (segment (start 78.994 72.8718) (end 78.994 83.616) (width 3.81) (layer "F.Cu") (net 4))
 (via (at 57.15 70.612) (size 1.524) (drill 0.762) (layers "F.Cu" "B.Cu") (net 4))
 (via (at 66.167 82.169) (size 1.524) (drill 0.762) (layers "F.Cu" "B.Cu") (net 4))
 (segment (start 78.295 87.693) (end 78.295 92.837) (width 2.54) (layer "B.Cu") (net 4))
 (segment (start 67.945 82.169) (end 70.358 79.756) (width 0.762) (layer "B.Cu") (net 4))
 (segment (start 66.167 82.169) (end 67.945 82.169) (width 0.762) (layer "B.Cu") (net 4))
 (segment (start 70.358 79.756) (end 78.295 87.693) (width 2.54) (layer "B.Cu") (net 4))
 (segment (start 57.15 70.612) (end 61.214 70.612) (width 0.762) (layer "B.Cu") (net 4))
 (segment (start 61.214 70.612) (end 70.358 79.756) (width 2.54) (layer "B.Cu") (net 4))
 (segment (start 56.35 78.493) (end 58.794 78.493) (width 0.25) (layer "F.Cu") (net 3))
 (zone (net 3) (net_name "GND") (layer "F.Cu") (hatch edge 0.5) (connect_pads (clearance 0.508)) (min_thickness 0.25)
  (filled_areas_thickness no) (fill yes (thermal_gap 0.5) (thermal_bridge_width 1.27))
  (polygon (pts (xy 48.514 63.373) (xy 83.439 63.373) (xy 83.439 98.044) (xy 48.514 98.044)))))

